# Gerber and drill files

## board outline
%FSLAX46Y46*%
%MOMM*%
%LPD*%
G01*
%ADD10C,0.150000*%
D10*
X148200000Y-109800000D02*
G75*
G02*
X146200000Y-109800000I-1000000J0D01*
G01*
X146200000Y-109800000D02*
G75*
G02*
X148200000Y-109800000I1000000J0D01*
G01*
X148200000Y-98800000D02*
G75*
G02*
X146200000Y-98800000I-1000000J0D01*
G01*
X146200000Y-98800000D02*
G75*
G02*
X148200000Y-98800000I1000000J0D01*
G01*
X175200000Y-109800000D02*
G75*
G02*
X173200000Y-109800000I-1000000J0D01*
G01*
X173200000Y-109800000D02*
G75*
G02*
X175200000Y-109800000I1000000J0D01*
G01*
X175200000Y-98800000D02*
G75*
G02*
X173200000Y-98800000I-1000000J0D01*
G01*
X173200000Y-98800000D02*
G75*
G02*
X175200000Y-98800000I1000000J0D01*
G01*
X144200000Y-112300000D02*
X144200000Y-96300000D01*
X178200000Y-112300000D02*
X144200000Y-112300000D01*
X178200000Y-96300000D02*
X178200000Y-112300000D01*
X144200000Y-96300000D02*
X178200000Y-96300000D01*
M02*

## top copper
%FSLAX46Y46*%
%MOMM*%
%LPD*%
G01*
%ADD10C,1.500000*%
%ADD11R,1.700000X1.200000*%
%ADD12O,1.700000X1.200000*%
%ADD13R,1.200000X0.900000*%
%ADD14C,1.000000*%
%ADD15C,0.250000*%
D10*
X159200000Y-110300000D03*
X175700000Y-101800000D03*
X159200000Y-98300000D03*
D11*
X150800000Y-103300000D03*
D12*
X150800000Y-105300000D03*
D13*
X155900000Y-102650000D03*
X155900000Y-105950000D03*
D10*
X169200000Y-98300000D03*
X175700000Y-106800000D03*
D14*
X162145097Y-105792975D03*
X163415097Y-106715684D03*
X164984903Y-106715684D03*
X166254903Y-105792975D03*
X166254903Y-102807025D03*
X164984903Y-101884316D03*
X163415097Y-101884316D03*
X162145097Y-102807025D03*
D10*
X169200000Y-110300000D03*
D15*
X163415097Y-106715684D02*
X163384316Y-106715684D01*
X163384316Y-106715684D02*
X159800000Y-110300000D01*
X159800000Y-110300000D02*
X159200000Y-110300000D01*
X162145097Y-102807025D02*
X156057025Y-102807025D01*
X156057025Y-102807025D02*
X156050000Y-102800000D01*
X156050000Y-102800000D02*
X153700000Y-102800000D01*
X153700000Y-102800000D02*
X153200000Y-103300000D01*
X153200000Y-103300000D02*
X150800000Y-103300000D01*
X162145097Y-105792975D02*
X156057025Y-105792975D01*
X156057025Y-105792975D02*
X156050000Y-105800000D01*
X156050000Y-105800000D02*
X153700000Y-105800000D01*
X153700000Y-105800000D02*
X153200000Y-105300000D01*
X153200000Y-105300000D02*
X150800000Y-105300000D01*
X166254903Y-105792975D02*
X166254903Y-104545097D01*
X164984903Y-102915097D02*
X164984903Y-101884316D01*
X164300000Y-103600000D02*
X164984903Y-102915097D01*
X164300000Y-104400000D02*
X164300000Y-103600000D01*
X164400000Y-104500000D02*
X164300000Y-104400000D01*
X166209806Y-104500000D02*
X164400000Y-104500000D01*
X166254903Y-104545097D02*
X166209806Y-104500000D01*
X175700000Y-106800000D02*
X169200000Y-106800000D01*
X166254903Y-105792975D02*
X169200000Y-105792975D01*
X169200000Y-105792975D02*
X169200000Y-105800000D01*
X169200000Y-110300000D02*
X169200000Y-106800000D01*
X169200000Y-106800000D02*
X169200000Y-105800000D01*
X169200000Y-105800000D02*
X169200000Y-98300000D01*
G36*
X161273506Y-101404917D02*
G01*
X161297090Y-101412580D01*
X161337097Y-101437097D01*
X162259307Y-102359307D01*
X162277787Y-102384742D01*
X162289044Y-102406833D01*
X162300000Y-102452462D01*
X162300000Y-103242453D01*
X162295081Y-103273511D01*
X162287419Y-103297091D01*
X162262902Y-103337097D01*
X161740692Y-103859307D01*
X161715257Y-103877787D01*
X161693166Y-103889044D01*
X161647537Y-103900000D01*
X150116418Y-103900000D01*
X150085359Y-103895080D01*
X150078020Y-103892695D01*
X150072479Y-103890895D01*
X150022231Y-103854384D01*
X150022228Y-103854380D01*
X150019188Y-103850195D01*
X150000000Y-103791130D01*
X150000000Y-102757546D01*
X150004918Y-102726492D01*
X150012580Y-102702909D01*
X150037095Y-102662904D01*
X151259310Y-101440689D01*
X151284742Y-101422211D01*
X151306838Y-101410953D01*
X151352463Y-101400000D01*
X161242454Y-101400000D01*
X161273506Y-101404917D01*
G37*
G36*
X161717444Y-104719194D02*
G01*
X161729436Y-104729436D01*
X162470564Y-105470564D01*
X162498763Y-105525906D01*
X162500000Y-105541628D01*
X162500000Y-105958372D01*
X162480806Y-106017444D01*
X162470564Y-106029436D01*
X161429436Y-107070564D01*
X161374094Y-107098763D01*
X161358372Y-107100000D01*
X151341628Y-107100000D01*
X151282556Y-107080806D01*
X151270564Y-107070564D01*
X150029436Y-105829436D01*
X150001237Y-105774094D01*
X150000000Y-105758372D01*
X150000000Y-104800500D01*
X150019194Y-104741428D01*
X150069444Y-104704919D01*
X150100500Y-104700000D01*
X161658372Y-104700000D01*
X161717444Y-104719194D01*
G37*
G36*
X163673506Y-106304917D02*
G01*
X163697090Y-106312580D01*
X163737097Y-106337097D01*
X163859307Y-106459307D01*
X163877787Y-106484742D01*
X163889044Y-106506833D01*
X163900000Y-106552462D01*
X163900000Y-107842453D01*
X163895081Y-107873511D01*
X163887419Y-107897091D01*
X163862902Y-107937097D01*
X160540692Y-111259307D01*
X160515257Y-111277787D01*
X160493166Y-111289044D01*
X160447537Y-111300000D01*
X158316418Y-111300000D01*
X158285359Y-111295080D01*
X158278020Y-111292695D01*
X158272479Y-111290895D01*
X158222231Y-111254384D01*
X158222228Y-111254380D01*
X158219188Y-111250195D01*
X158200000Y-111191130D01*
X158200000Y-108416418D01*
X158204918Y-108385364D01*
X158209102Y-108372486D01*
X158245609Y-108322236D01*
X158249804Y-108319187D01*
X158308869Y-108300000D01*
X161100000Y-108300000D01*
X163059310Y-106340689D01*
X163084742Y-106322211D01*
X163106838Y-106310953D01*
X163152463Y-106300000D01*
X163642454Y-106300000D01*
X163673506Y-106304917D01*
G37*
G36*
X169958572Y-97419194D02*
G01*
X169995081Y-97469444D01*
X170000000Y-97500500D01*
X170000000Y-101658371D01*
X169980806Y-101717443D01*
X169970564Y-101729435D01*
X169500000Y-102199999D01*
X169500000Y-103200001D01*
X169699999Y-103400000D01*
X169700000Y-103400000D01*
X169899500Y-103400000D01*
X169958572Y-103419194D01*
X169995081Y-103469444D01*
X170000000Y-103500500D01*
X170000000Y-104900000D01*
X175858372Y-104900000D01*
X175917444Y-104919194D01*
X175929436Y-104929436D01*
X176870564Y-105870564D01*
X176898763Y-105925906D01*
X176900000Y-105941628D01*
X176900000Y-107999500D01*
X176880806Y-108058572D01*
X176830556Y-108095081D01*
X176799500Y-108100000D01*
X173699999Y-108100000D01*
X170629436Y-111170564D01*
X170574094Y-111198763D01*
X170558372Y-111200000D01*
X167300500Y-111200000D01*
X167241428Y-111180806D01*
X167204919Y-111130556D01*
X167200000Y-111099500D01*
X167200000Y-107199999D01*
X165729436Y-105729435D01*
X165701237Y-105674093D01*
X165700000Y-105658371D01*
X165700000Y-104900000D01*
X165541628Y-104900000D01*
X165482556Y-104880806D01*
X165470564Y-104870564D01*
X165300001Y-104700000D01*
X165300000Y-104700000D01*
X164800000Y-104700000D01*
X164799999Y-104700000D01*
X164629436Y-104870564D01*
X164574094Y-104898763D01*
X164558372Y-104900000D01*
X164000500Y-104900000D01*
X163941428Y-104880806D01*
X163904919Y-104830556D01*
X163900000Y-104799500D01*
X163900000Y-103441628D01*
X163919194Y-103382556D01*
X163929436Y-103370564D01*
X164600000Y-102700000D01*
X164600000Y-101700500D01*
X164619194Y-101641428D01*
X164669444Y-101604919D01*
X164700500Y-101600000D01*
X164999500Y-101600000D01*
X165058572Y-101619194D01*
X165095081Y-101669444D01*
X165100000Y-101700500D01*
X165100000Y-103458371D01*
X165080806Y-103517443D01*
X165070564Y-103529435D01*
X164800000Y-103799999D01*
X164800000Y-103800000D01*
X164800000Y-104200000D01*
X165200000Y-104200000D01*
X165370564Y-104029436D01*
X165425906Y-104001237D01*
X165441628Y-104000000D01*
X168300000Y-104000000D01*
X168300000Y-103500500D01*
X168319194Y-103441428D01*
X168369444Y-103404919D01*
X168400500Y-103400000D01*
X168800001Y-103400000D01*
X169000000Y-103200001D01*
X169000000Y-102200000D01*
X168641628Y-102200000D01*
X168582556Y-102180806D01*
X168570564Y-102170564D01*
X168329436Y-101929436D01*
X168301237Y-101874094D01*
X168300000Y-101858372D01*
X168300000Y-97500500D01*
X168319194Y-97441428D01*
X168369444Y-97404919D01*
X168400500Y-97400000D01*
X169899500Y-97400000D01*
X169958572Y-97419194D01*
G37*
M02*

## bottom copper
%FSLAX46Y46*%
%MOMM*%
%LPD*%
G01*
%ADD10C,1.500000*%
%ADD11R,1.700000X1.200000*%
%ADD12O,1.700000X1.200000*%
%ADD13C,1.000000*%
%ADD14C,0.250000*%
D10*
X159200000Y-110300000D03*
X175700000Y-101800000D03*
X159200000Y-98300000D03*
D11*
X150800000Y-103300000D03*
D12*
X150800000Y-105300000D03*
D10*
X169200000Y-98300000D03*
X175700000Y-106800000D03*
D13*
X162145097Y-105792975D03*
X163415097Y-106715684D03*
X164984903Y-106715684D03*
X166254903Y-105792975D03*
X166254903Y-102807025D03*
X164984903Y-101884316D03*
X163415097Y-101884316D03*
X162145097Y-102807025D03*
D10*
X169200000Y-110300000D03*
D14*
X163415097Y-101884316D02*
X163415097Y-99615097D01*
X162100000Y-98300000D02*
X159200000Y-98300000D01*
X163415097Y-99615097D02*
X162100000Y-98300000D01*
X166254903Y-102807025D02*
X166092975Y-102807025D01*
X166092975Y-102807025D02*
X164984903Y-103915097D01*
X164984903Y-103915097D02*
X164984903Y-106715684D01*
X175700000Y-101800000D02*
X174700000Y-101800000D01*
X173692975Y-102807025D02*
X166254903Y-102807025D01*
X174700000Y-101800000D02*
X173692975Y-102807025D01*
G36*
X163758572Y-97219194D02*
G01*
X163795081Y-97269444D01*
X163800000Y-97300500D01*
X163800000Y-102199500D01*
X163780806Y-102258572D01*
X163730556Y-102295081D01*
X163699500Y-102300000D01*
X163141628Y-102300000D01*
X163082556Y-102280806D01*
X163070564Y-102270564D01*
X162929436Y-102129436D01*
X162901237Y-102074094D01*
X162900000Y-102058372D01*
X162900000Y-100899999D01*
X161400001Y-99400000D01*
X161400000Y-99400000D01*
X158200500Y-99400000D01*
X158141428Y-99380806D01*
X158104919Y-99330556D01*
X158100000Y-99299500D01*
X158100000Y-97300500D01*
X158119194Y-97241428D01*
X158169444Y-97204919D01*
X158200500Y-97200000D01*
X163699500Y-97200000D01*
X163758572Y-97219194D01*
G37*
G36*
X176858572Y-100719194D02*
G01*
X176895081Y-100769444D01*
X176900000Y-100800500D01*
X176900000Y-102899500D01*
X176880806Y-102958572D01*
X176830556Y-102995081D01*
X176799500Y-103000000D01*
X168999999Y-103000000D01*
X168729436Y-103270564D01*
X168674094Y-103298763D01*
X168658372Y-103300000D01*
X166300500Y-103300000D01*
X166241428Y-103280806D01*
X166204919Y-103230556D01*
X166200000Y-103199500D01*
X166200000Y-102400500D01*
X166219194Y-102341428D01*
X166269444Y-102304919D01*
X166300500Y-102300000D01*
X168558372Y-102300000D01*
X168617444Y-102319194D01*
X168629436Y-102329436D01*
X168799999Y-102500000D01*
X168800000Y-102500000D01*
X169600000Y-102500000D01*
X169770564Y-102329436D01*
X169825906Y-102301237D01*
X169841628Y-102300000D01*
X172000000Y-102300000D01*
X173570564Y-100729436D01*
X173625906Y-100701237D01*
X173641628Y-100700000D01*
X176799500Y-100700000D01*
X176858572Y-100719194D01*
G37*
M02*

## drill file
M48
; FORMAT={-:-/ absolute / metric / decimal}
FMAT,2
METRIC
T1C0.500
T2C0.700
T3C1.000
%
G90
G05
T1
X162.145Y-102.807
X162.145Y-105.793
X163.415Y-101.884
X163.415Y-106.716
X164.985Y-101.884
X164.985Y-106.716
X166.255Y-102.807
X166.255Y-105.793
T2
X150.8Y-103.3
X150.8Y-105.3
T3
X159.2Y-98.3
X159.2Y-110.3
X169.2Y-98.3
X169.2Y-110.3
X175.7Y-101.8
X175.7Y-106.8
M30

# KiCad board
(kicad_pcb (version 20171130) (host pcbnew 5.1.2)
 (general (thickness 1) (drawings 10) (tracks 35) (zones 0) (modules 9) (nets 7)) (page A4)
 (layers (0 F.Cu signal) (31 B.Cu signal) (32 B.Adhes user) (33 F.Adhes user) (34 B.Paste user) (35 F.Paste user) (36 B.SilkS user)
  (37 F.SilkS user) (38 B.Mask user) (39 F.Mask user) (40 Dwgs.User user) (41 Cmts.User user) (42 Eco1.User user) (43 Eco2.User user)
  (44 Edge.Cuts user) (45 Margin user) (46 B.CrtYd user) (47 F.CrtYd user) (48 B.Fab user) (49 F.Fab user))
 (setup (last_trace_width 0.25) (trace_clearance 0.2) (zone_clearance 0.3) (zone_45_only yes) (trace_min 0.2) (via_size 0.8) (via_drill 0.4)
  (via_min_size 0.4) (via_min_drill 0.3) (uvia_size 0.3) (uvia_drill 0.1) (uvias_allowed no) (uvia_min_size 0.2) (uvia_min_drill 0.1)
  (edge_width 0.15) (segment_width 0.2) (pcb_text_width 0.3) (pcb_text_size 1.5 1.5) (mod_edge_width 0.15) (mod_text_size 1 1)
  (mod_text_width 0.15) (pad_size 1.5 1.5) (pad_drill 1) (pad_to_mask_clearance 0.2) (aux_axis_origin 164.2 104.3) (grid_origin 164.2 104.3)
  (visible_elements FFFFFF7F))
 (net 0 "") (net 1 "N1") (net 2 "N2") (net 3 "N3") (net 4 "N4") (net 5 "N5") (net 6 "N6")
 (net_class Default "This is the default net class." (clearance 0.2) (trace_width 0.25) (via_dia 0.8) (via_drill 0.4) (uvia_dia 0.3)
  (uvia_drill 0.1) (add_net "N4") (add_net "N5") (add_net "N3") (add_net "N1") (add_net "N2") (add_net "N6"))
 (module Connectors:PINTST (layer F.Cu) (at 159.2 110.3)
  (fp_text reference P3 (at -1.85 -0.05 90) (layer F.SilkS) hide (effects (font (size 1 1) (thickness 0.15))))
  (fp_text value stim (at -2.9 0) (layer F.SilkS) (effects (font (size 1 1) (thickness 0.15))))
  (pad 1 thru_hole circle (at 0 0) (size 1.5 1.5) (drill 1) (layers *.Cu *.Mask) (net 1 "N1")))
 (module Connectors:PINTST (layer F.Cu) (at 175.7 101.8)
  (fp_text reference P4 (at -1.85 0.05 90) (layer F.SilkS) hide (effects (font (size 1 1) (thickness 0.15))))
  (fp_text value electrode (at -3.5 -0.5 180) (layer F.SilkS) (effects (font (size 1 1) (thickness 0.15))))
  (pad 1 thru_hole circle (at 0 0) (size 1.5 1.5) (drill 1) (layers *.Cu *.Mask) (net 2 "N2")))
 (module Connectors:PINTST (layer F.Cu) (at 159.2 98.3)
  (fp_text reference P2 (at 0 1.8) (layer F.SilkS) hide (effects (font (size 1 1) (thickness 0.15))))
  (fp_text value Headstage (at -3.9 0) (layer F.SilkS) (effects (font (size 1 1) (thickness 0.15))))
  (pad 1 thru_hole circle (at 0 0) (size 1.5 1.5) (drill 1) (layers *.Cu *.Mask) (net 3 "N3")))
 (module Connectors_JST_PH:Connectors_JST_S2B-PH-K (layer F.Cu) (at 150.8 103.3 270)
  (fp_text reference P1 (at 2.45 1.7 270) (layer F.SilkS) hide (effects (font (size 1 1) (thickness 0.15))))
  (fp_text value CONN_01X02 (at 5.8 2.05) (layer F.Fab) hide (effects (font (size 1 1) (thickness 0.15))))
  (pad 1 thru_hole rect (at 0 0 270) (size 1.2 1.7) (drill 0.7) (layers *.Cu *.Mask F.SilkS) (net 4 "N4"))
  (pad 2 thru_hole oval (at 2 0 270) (size 1.2 1.7) (drill 0.7) (layers *.Cu *.Mask F.SilkS) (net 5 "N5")))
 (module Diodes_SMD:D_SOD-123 (layer F.Cu) (at 155.9 104.3 270)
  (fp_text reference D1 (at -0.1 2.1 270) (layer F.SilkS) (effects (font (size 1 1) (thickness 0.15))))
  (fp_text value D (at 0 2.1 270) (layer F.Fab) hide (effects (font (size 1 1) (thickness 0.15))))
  (pad 1 smd rect (at -1.65 0 270) (size 0.9 1.2) (layers F.Cu F.Paste F.Mask) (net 4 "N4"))
  (pad 2 smd rect (at 1.65 0 270) (size 0.9 1.2) (layers F.Cu F.Paste F.Mask) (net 5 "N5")))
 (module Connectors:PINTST (layer F.Cu) (at 169.2 98.3)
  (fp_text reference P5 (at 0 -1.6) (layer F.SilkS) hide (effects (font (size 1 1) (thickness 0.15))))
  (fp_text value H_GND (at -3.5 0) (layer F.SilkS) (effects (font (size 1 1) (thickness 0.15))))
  (pad 1 thru_hole circle (at 0 0) (size 1.5 1.5) (drill 1) (layers *.Cu *.Mask) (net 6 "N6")))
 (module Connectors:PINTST (layer F.Cu) (at 175.7 106.8)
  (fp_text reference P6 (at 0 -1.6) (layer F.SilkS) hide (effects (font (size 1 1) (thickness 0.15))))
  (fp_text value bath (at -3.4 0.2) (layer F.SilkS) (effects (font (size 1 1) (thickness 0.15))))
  (pad 1 thru_hole circle (at 0 0) (size 1.5 1.5) (drill 1) (layers *.Cu *.Mask) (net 6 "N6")))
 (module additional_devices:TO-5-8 (layer F.Cu) (at 164.2 104.3 90)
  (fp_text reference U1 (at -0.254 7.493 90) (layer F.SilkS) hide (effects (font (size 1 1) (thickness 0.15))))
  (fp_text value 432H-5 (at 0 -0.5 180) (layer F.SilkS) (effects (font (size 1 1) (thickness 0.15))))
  (pad 8 thru_hole circle (at -1.492975 -2.054903 162) (size 1 1) (drill 0.5) (layers *.Cu *.Mask) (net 5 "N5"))
  (pad 7 thru_hole circle (at -2.415684 -0.784903 198) (size 1 1) (drill 0.5) (layers *.Cu *.Mask) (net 1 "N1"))
  (pad 6 thru_hole circle (at -2.415684 0.784903 234) (size 1 1) (drill 0.5) (layers *.Cu *.Mask) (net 2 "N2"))
  (pad 5 thru_hole circle (at -1.492975 2.054903 270) (size 1 1) (drill 0.5) (layers *.Cu *.Mask) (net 6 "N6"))
  (pad 4 thru_hole circle (at 1.492975 2.054903 342) (size 1 1) (drill 0.5) (layers *.Cu *.Mask) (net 2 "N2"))
  (pad 3 thru_hole circle (at 2.415684 0.784903 18) (size 1 1) (drill 0.5) (layers *.Cu *.Mask) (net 6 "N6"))
  (pad 2 thru_hole circle (at 2.415684 -0.784903 54) (size 1 1) (drill 0.5) (layers *.Cu *.Mask) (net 3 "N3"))
  (pad 1 thru_hole circle (at 1.492975 -2.054903 90) (size 1 1) (drill 0.5) (layers *.Cu *.Mask) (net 4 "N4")))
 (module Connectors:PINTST (layer F.Cu) (at 169.2 110.3)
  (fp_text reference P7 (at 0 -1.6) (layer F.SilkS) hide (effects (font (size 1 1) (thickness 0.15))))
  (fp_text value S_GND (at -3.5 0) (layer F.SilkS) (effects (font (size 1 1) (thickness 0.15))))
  (pad 1 thru_hole circle (at 0 0) (size 1.5 1.5) (drill 1) (layers *.Cu *.Mask) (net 6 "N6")))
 (gr_circle (center 147.2 109.8) (end 148.2 109.8) (layer Edge.Cuts) (width 0.15))
 (gr_circle (center 147.2 98.8) (end 148.2 98.8) (layer Edge.Cuts) (width 0.15))
 (gr_circle (center 174.2 109.8) (end 175.2 109.8) (layer Edge.Cuts) (width 0.15))
 (gr_circle (center 174.2 98.8) (end 175.2 98.8) (layer Edge.Cuts) (width 0.15))
 (gr_line (start 144.2 112.3) (end 144.2 96.3) (angle 90) (layer Edge.Cuts) (width 0.15))
 (gr_line (start 178.2 112.3) (end 144.2 112.3) (angle 90) (layer Edge.Cuts) (width 0.15))
 (gr_line (start 178.2 96.3) (end 178.2 112.3) (angle 90) (layer Edge.Cuts) (width 0.15))
 (gr_line (start 144.2 96.3) (end 178.2 96.3) (angle 90) (layer Edge.Cuts) (width 0.15))
 (segment (start 163.415097 101.884316) (end 163.415097 99.615097) (width 0.25) (layer B.Cu) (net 3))
 (segment (start 162.1 98.3) (end 159.2 98.3) (width 0.25) (layer B.Cu) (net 3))
 (segment (start 163.415097 99.615097) (end 162.1 98.3) (width 0.25) (layer B.Cu) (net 3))
 (segment (start 163.415097 106.715684) (end 163.384316 106.715684) (width 0.25) (layer F.Cu) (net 1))
 (segment (start 163.384316 106.715684) (end 159.8 110.3) (width 0.25) (layer F.Cu) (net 1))
 (segment (start 159.8 110.3) (end 159.2 110.3) (width 0.25) (layer F.Cu) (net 1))
 (segment (start 166.254903 102.807025) (end 166.092975 102.807025) (width 0.25) (layer B.Cu) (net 2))
 (segment (start 166.092975 102.807025) (end 164.984903 103.915097) (width 0.25) (layer B.Cu) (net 2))
 (segment (start 164.984903 103.915097) (end 164.984903 106.715684) (width 0.25) (layer B.Cu) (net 2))
 (segment (start 175.7 101.8) (end 174.7 101.8) (width 0.25) (layer B.Cu) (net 2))
 (segment (start 173.692975 102.807025) (end 166.254903 102.807025) (width 0.25) (layer B.Cu) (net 2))
 (segment (start 174.7 101.8) (end 173.692975 102.807025) (width 0.25) (layer B.Cu) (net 2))
 (segment (start 162.145097 102.807025) (end 156.057025 102.807025) (width 0.25) (layer F.Cu) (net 4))
 (segment (start 156.057025 102.807025) (end 156.05 102.8) (width 0.25) (layer F.Cu) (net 4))
 (segment (start 156.05 102.8) (end 153.7 102.8) (width 0.25) (layer F.Cu) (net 4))
 (segment (start 153.7 102.8) (end 153.2 103.3) (width 0.25) (layer F.Cu) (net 4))
 (segment (start 153.2 103.3) (end 150.8 103.3) (width 0.25) (layer F.Cu) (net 4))
 (segment (start 162.145097 105.792975) (end 156.057025 105.792975) (width 0.25) (layer F.Cu) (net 5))
 (segment (start 156.057025 105.792975) (end 156.05 105.8) (width 0.25) (layer F.Cu) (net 5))
 (segment (start 156.05 105.8) (end 153.7 105.8) (width 0.25) (layer F.Cu) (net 5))
 (segment (start 153.7 105.8) (end 153.2 105.3) (width 0.25) (layer F.Cu) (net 5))
 (segment (start 153.2 105.3) (end 150.8 105.3) (width 0.25) (layer F.Cu) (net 5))
 (segment (start 166.254903 105.792975) (end 166.254903 104.545097) (width 0.25) (layer F.Cu) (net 6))
 (segment (start 164.984903 102.915097) (end 164.984903 101.884316) (width 0.25) (layer F.Cu) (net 6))
 (segment (start 164.3 103.6) (end 164.984903 102.915097) (width 0.25) (layer F.Cu) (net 6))
 (segment (start 164.3 104.4) (end 164.3 103.6) (width 0.25) (layer F.Cu) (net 6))
 (segment (start 164.4 104.5) (end 164.3 104.4) (width 0.25) (layer F.Cu) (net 6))
 (segment (start 166.209806 104.5) (end 164.4 104.5) (width 0.25) (layer F.Cu) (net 6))
 (segment (start 166.254903 104.545097) (end 166.209806 104.5) (width 0.25) (layer F.Cu) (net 6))
 (segment (start 175.7 106.8) (end 169.2 106.8) (width 0.25) (layer F.Cu) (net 6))
 (segment (start 166.254903 105.792975) (end 169.2 105.792975) (width 0.25) (layer F.Cu) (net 6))
 (segment (start 169.2 105.792975) (end 169.2 105.8) (width 0.25) (layer F.Cu) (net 6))
 (segment (start 169.2 110.3) (end 169.2 106.8) (width 0.25) (layer F.Cu) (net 6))
 (segment (start 169.2 106.8) (end 169.2 105.8) (width 0.25) (layer F.Cu) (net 6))
 (segment (start 169.2 105.8) (end 169.2 98.3) (width 0.25) (layer F.Cu) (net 6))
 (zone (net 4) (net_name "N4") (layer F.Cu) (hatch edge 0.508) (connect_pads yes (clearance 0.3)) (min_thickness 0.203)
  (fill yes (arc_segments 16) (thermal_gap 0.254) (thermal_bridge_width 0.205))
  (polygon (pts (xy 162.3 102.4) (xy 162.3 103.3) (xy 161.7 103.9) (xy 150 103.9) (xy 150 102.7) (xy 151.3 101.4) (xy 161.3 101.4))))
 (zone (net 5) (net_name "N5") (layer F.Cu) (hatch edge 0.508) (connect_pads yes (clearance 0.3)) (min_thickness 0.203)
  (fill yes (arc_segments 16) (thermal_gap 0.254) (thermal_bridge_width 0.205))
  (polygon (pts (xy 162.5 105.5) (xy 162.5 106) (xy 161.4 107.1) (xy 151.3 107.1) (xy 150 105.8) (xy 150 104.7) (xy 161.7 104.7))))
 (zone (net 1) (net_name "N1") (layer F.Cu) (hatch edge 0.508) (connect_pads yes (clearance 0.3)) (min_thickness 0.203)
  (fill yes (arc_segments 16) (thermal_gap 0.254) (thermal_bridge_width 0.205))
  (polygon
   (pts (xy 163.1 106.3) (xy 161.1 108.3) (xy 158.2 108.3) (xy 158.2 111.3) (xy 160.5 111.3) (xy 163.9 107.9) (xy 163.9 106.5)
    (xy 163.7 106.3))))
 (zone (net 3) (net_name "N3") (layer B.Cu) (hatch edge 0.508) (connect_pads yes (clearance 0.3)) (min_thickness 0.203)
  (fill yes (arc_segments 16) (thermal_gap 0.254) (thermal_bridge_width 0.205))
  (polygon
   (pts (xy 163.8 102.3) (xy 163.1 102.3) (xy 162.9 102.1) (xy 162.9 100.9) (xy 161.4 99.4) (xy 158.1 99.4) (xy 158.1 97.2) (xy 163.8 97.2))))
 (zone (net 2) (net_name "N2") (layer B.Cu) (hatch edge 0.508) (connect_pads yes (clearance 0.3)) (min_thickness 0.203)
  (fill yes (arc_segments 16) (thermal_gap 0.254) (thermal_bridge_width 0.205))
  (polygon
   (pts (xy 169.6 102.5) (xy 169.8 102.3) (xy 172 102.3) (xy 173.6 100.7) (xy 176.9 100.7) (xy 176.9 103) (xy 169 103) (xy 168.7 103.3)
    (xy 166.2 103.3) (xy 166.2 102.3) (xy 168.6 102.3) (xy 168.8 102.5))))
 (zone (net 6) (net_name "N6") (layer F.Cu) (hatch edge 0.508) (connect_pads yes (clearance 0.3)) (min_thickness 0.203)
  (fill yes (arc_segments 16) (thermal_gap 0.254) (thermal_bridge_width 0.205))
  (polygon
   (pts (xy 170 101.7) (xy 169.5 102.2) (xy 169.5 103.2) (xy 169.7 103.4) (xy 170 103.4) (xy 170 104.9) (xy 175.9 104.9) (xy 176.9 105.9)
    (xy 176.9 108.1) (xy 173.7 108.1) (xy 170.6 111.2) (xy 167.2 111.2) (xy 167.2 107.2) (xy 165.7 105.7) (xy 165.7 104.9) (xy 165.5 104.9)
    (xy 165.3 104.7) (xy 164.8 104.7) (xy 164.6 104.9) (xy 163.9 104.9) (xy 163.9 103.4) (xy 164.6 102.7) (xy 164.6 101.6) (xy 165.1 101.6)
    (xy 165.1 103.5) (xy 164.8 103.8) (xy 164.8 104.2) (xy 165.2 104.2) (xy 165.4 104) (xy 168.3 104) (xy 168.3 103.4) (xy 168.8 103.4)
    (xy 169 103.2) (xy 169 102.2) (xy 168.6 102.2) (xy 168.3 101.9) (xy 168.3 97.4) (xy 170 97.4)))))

